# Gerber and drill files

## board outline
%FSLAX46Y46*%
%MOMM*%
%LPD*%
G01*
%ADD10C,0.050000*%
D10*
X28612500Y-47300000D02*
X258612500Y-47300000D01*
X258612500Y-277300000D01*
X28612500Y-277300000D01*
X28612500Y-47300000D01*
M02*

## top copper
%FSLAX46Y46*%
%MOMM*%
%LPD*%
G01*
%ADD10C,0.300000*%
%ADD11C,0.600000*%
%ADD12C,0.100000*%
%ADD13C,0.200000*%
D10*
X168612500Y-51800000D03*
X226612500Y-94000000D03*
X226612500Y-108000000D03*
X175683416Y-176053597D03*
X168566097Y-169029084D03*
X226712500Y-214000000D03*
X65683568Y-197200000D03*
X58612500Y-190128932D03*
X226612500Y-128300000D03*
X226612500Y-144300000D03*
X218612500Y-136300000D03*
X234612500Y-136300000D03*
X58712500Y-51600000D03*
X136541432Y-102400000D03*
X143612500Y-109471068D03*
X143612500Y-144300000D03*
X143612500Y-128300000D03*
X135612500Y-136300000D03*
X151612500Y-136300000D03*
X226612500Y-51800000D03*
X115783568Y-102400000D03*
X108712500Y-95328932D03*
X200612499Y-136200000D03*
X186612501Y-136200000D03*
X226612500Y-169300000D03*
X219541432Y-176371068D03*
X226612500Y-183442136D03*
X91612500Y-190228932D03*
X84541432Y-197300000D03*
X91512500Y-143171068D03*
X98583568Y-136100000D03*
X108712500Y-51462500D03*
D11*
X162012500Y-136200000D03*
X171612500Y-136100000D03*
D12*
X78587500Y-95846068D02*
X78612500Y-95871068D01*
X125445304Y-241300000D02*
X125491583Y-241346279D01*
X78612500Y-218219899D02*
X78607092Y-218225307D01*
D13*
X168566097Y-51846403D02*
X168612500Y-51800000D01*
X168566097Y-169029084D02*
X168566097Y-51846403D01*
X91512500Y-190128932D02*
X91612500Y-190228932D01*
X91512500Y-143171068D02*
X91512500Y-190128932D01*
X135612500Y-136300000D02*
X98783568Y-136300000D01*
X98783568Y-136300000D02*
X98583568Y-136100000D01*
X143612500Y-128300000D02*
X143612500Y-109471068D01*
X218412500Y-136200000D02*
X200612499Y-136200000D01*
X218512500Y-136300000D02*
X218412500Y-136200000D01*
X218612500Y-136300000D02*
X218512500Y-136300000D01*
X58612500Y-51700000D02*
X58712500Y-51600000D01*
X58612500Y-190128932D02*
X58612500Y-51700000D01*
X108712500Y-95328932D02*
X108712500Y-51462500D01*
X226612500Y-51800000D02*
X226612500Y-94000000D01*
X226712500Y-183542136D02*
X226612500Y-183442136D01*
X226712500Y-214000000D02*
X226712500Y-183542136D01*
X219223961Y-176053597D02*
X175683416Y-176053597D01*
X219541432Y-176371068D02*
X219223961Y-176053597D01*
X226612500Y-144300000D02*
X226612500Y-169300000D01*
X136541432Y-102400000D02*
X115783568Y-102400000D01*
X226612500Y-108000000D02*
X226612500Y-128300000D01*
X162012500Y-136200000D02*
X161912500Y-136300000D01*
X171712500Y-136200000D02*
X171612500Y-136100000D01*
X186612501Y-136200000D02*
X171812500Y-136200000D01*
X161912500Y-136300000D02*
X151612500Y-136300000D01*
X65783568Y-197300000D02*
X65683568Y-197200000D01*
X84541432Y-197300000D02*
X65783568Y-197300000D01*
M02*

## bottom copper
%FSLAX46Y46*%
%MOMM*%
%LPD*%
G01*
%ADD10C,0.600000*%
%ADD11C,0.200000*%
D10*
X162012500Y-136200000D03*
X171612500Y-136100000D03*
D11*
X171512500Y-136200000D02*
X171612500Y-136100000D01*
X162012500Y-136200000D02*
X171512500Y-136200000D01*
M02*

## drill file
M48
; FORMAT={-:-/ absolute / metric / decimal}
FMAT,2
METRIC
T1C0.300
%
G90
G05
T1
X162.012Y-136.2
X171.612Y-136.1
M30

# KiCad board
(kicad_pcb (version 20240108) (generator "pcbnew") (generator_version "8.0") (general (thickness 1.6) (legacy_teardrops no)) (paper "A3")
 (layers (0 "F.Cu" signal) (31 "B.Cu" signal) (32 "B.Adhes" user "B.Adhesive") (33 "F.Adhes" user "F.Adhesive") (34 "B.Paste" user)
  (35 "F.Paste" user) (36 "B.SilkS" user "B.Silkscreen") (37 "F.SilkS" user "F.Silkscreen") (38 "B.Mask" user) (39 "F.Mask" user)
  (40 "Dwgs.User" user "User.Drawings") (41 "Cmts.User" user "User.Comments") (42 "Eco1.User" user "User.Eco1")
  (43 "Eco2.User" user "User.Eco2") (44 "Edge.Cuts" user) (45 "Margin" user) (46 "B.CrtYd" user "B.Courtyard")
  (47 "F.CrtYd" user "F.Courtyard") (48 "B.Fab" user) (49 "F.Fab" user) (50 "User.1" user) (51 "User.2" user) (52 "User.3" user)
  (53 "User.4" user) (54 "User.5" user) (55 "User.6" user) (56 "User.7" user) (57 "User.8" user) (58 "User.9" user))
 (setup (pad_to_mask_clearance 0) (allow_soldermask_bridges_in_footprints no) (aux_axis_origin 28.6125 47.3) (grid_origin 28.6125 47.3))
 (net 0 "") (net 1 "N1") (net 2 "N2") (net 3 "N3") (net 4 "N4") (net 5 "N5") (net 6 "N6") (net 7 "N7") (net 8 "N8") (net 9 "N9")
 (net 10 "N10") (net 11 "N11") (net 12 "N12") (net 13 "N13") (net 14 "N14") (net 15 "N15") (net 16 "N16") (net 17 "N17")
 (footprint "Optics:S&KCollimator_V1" (layer "F.Cu") (at 168.6125 51.8 -90)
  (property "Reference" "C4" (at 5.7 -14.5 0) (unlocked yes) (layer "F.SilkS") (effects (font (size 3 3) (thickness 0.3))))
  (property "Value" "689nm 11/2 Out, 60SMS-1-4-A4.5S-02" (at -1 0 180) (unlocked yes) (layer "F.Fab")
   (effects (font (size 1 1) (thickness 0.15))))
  (pad "1" smd circle (at 0 0 180) (size 0.3 0.3) (layers "F.Cu" "F.Paste" "F.Mask") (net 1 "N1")))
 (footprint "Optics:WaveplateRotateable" (layer "F.Cu") (at 226.6125 101)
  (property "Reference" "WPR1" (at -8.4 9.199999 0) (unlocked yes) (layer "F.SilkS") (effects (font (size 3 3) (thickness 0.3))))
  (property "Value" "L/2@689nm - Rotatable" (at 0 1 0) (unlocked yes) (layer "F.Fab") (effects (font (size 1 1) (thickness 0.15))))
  (pad "1" smd circle (at 0 -7) (size 0.3 0.3) (layers "F.Cu" "F.Paste" "F.Mask") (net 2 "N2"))
  (pad "2" smd circle (at 0 7) (size 0.3 0.3) (layers "F.Cu" "F.Paste" "F.Mask") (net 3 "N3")))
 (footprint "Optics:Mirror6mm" (layer "F.Cu") (at 168.6125 176.1 45.376)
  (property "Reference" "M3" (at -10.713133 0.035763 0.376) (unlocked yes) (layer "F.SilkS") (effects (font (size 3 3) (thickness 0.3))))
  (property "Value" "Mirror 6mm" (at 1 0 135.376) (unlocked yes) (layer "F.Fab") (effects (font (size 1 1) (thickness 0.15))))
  (pad "1" smd circle (at 5 5 135.376) (size 0.3 0.3) (layers "F.Cu" "F.Paste" "F.Mask") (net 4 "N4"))
  (pad "2" smd circle (at 5 -5 135.376) (size 0.3 0.3) (layers "F.Cu" "F.Paste" "F.Mask") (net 1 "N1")))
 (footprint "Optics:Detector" (layer "F.Cu") (at 226.7125 219)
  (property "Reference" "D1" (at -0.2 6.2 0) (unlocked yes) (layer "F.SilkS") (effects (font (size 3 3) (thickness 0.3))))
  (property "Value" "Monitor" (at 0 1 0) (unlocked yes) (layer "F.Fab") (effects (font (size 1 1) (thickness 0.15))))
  (pad "1" smd circle (at 0 -5 180) (size 0.3 0.3) (layers "F.Cu" "F.Paste" "F.Mask") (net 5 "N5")))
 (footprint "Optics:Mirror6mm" (layer "F.Cu") (at 58.6125 197.2 45)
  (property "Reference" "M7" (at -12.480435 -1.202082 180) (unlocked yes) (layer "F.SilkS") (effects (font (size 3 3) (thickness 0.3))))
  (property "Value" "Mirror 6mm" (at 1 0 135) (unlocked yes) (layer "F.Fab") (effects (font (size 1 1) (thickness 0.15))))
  (pad "1" smd circle (at 5 5 135) (size 0.3 0.3) (layers "F.Cu" "F.Paste" "F.Mask") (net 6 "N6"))
  (pad "2" smd circle (at 5 -5 135) (size 0.3 0.3) (layers "F.Cu" "F.Paste" "F.Mask") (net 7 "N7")))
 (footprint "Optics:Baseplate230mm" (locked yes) (layer "F.Cu") (at 28.6125 47.3)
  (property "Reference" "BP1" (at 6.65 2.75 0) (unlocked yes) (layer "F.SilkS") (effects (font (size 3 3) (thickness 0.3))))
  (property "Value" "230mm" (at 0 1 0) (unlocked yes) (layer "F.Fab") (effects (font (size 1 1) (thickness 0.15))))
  (fp_rect (start 0 0) (end 230 230) (stroke (width 0.05) (type default)) (fill none) (layer "Edge.Cuts")))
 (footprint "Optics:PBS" (layer "F.Cu") (at 226.6125 136.3 -90)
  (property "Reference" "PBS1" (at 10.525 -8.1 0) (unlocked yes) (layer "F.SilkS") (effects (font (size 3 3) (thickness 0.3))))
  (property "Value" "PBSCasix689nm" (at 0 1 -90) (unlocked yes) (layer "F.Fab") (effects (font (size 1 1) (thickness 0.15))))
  (pad "1" smd circle (at -8 0 270) (size 0.3 0.3) (layers "F.Cu" "F.Paste" "F.Mask") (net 3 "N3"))
  (pad "2" smd circle (at 8 0 270) (size 0.3 0.3) (layers "F.Cu" "F.Paste" "F.Mask") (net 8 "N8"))
  (pad "3" smd circle (at 0 8 270) (size 0.3 0.3) (layers "F.Cu" "F.Paste" "F.Mask") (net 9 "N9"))
  (pad "4" smd circle (at 0 -8 270) (size 0.3 0.3) (layers "F.Cu" "F.Paste" "F.Mask") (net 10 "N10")))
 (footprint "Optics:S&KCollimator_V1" (layer "F.Cu") (at 58.7125 51.6 -90)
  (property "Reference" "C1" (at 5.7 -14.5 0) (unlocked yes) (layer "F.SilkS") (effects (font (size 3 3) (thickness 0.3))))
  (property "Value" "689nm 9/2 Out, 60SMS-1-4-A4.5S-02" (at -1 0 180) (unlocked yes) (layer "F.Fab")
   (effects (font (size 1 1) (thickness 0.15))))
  (pad "1" smd circle (at 0 0 180) (size 0.3 0.3) (layers "F.Cu" "F.Paste" "F.Mask") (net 7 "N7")))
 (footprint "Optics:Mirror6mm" (layer "F.Cu") (at 143.6125 102.4 -135)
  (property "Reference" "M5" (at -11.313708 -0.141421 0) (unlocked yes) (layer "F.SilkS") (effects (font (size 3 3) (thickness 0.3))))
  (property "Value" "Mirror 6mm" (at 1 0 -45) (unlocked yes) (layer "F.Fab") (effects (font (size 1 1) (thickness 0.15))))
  (pad "1" smd circle (at 5 5 315) (size 0.3 0.3) (layers "F.Cu" "F.Paste" "F.Mask") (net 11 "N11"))
  (pad "2" smd circle (at 5 -5 315) (size 0.3 0.3) (layers "F.Cu" "F.Paste" "F.Mask") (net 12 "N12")))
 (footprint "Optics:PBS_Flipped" (layer "F.Cu") (at 143.6125 136.3 -90)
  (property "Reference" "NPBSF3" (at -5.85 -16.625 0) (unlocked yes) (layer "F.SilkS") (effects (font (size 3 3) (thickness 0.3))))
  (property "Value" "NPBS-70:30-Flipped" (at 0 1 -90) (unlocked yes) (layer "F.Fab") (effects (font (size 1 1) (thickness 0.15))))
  (pad "1" smd circle (at 8 0 90) (size 0.3 0.3) (layers "F.Cu" "F.Paste" "F.Mask") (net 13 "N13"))
  (pad "2" smd circle (at -8 0 90) (size 0.3 0.3) (layers "F.Cu" "F.Paste" "F.Mask") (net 12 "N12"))
  (pad "3" smd circle (at 0 8 270) (size 0.3 0.3) (layers "F.Cu" "F.Paste" "F.Mask") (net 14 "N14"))
  (pad "4" smd circle (at 0 -8 270) (size 0.3 0.3) (layers "F.Cu" "F.Paste" "F.Mask") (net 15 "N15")))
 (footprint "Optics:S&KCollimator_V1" (layer "F.Cu") (at 226.6125 51.8 -90)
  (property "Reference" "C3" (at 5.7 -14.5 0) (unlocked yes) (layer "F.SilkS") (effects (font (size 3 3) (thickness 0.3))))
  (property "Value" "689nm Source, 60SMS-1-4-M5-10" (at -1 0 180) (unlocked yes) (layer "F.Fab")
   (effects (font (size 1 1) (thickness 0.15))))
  (pad "1" smd circle (at 0 0 180) (size 0.3 0.3) (layers "F.Cu" "F.Paste" "F.Mask") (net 2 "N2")))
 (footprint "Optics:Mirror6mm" (layer "F.Cu") (at 108.7125 102.4 45)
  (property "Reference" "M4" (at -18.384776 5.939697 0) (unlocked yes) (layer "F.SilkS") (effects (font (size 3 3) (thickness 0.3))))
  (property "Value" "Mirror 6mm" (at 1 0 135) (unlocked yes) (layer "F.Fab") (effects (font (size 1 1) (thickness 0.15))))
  (pad "1" smd circle (at 5 5 135) (size 0.3 0.3) (layers "F.Cu" "F.Paste" "F.Mask") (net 11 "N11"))
  (pad "2" smd circle (at 5 -5 135) (size 0.3 0.3) (layers "F.Cu" "F.Paste" "F.Mask") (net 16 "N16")))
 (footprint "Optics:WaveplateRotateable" (layer "F.Cu") (at 193.6125 136.2 -90)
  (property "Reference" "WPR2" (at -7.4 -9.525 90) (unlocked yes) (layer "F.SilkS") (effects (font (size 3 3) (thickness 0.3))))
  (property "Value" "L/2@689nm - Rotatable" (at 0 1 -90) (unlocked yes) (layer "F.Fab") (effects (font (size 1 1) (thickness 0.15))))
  (pad "1" smd circle (at 0 -6.999999 270) (size 0.3 0.3) (layers "F.Cu" "F.Paste" "F.Mask") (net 9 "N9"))
  (pad "2" smd circle (at 0 6.999999 270) (size 0.3 0.3) (layers "F.Cu" "F.Paste" "F.Mask") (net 15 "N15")))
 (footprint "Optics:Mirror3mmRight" (layer "F.Cu") (at 226.6125 176.371068 135)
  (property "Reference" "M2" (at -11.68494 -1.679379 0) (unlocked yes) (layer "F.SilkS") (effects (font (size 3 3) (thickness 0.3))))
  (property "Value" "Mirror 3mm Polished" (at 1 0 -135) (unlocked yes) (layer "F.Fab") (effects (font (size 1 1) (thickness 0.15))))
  (pad "1" smd circle (at 5 5 225) (size 0.3 0.3) (layers "F.Cu" "F.Paste" "F.Mask") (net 8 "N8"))
  (pad "2" smd circle (at 5 -5 225) (size 0.3 0.3) (layers "F.Cu" "F.Paste" "F.Mask") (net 4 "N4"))
  (pad "3" smd circle (at -5 -5 225) (size 0.3 0.3) (layers "F.Cu" "F.Paste" "F.Mask") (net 5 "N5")))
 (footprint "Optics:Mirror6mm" (layer "F.Cu") (at 91.6125 197.3 135)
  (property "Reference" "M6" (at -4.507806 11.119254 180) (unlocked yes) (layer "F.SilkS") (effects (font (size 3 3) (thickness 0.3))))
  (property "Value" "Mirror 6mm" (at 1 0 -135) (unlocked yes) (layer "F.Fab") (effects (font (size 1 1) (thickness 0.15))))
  (pad "1" smd circle (at 5 5 225) (size 0.3 0.3) (layers "F.Cu" "F.Paste" "F.Mask") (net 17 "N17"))
  (pad "2" smd circle (at 5 -5 225) (size 0.3 0.3) (layers "F.Cu" "F.Paste" "F.Mask") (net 6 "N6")))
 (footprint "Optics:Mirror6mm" (layer "F.Cu") (at 91.5125 136.1 -45)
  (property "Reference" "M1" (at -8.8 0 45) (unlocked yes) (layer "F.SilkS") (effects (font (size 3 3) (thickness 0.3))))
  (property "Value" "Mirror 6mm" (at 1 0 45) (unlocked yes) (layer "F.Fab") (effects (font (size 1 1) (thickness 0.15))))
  (pad "1" smd circle (at 5 5 45) (size 0.3 0.3) (layers "F.Cu" "F.Paste" "F.Mask") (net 17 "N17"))
  (pad "2" smd circle (at 5 -5 45) (size 0.3 0.3) (layers "F.Cu" "F.Paste" "F.Mask") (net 14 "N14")))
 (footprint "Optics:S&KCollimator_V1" (layer "F.Cu") (at 108.7125 51.4625 -90)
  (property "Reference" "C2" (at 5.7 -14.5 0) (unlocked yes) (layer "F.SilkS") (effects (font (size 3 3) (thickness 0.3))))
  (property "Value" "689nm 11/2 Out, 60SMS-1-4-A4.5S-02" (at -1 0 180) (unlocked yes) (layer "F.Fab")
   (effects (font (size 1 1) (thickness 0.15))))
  (pad "1" smd circle (at 0 0 180) (size 0.3 0.3) (layers "F.Cu" "F.Paste" "F.Mask") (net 16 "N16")))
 (segment (start 78.5875 95.846068) (end 78.6125 95.871068) (width 0.1) (layer "F.Cu") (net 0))
 (segment (start 125.445304 241.3) (end 125.491583 241.346279) (width 0.1) (layer "F.Cu") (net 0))
 (segment (start 78.6125 218.219899) (end 78.607092 218.225307) (width 0.1) (layer "F.Cu") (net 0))
 (segment (start 168.566097 51.846403) (end 168.6125 51.8) (width 0.2) (layer "F.Cu") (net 1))
 (segment (start 168.566097 169.029084) (end 168.566097 51.846403) (width 0.2) (layer "F.Cu") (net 1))
 (segment (start 91.5125 190.128932) (end 91.6125 190.228932) (width 0.2) (layer "F.Cu") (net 17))
 (segment (start 91.5125 143.171068) (end 91.5125 190.128932) (width 0.2) (layer "F.Cu") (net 17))
 (segment (start 135.6125 136.3) (end 98.783568 136.3) (width 0.2) (layer "F.Cu") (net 14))
 (segment (start 98.783568 136.3) (end 98.583568 136.1) (width 0.2) (layer "F.Cu") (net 14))
 (segment (start 143.6125 128.3) (end 143.6125 109.471068) (width 0.2) (layer "F.Cu") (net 12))
 (segment (start 218.4125 136.2) (end 200.612499 136.2) (width 0.2) (layer "F.Cu") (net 9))
 (segment (start 218.5125 136.3) (end 218.4125 136.2) (width 0.2) (layer "F.Cu") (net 9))
 (segment (start 218.6125 136.3) (end 218.5125 136.3) (width 0.2) (layer "F.Cu") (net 9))
 (segment (start 58.6125 51.7) (end 58.7125 51.6) (width 0.2) (layer "F.Cu") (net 7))
 (segment (start 58.6125 190.128932) (end 58.6125 51.7) (width 0.2) (layer "F.Cu") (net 7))
 (segment (start 108.7125 95.328932) (end 108.7125 51.4625) (width 0.2) (layer "F.Cu") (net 16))
 (segment (start 226.6125 51.8) (end 226.6125 94) (width 0.2) (layer "F.Cu") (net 2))
 (segment (start 226.7125 183.542136) (end 226.6125 183.442136) (width 0.2) (layer "F.Cu") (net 5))
 (segment (start 226.7125 214) (end 226.7125 183.542136) (width 0.2) (layer "F.Cu") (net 5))
 (segment (start 219.223961 176.053597) (end 175.683416 176.053597) (width 0.2) (layer "F.Cu") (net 4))
 (segment (start 219.541432 176.371068) (end 219.223961 176.053597) (width 0.2) (layer "F.Cu") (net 4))
 (segment (start 226.6125 144.3) (end 226.6125 169.3) (width 0.2) (layer "F.Cu") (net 8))
 (segment (start 136.541432 102.4) (end 115.783568 102.4) (width 0.2) (layer "F.Cu") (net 11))
 (segment (start 226.6125 108) (end 226.6125 128.3) (width 0.2) (layer "F.Cu") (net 3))
 (segment (start 162.0125 136.2) (end 161.9125 136.3) (width 0.2) (layer "F.Cu") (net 15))
 (segment (start 171.7125 136.2) (end 171.6125 136.1) (width 0.2) (layer "F.Cu") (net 15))
 (segment (start 186.612501 136.2) (end 171.8125 136.2) (width 0.2) (layer "F.Cu") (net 15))
 (segment (start 161.9125 136.3) (end 151.6125 136.3) (width 0.2) (layer "F.Cu") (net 15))
 (via (at 162.0125 136.2) (size 0.6) (drill 0.3) (layers "F.Cu" "B.Cu") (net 15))
 (via (at 171.6125 136.1) (size 0.6) (drill 0.3) (layers "F.Cu" "B.Cu") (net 15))
 (segment (start 171.5125 136.2) (end 171.6125 136.1) (width 0.2) (layer "B.Cu") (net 15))
 (segment (start 162.0125 136.2) (end 171.5125 136.2) (width 0.2) (layer "B.Cu") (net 15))
 (segment (start 65.783568 197.3) (end 65.683568 197.2) (width 0.2) (layer "F.Cu") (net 6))
 (segment (start 84.541432 197.3) (end 65.783568 197.3) (width 0.2) (layer "F.Cu") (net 6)))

